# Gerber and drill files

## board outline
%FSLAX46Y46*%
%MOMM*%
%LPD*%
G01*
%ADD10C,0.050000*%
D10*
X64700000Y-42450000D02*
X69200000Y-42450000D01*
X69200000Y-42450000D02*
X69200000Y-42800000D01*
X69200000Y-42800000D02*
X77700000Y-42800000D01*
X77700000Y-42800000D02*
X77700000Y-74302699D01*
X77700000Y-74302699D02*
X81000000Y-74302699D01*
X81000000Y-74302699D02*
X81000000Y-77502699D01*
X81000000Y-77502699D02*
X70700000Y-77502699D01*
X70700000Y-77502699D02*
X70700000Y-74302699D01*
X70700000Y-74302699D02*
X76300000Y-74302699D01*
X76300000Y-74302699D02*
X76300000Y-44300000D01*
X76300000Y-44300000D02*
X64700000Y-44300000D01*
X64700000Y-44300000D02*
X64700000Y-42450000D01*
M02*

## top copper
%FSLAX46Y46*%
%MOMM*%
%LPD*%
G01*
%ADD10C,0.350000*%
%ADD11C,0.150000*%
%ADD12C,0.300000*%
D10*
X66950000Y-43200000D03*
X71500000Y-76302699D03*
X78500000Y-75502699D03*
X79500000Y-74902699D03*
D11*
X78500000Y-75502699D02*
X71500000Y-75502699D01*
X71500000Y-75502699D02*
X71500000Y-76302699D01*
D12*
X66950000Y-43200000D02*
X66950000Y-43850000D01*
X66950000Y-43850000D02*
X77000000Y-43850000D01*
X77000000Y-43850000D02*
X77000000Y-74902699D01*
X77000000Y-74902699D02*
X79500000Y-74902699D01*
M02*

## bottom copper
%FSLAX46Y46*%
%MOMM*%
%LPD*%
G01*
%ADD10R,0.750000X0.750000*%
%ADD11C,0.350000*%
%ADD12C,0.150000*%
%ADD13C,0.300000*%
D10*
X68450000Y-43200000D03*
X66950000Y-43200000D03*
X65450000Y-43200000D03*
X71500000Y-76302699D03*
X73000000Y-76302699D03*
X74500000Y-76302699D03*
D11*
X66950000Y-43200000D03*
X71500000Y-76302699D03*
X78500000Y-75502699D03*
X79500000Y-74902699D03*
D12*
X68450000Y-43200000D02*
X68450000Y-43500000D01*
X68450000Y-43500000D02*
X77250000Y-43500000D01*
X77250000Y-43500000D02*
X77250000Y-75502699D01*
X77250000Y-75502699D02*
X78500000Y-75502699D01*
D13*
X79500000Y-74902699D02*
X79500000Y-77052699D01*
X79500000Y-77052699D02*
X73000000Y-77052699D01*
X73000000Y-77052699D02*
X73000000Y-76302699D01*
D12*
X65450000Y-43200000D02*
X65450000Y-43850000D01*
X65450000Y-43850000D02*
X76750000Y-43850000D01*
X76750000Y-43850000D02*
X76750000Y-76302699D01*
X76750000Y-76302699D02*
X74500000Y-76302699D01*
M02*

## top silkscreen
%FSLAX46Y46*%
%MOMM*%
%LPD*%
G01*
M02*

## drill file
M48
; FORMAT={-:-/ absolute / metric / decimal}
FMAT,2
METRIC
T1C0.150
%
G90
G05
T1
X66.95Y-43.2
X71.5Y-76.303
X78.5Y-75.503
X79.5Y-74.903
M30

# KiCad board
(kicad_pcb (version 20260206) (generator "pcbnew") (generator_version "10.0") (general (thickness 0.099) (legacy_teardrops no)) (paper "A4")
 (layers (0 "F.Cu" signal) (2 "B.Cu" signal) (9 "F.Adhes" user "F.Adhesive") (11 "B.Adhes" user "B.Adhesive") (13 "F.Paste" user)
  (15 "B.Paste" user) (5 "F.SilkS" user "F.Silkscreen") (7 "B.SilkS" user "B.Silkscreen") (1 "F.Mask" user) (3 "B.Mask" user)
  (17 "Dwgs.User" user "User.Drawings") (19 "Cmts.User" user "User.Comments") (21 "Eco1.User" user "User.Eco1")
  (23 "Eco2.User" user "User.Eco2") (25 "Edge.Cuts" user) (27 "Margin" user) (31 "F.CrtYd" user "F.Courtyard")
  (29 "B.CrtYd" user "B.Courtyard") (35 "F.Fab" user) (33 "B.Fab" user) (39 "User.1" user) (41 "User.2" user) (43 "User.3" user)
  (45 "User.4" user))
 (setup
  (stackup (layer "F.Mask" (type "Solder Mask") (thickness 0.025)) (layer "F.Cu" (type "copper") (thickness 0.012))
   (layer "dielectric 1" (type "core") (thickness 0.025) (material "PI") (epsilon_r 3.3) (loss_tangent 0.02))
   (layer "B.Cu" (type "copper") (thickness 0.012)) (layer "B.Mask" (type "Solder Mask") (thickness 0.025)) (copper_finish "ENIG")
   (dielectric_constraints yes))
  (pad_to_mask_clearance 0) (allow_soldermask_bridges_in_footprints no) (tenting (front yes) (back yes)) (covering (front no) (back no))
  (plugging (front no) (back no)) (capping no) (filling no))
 (gr_line (start 64.7 42.45000000000001) (end 69.2 42.45000000000001) (stroke (width 0.05) (type default)) (layer "Edge.Cuts"))
 (gr_line (start 69.2 42.45000000000001) (end 69.2 42.80000000000001) (stroke (width 0.05) (type default)) (layer "Edge.Cuts"))
 (gr_line (start 69.2 42.80000000000001) (end 77.7 42.80000000000001) (stroke (width 0.05) (type default)) (layer "Edge.Cuts"))
 (gr_line (start 77.7 42.80000000000001) (end 77.7 74.30269878025518) (stroke (width 0.05) (type default)) (layer "Edge.Cuts"))
 (gr_line (start 77.7 74.30269878025518) (end 81.0 74.30269878025518) (stroke (width 0.05) (type default)) (layer "Edge.Cuts"))
 (gr_line (start 81.0 74.30269878025518) (end 81.0 77.50269878025519) (stroke (width 0.05) (type default)) (layer "Edge.Cuts"))
 (gr_line (start 81.0 77.50269878025519) (end 70.7 77.50269878025519) (stroke (width 0.05) (type default)) (layer "Edge.Cuts"))
 (gr_line (start 70.7 77.50269878025519) (end 70.7 74.30269878025518) (stroke (width 0.05) (type default)) (layer "Edge.Cuts"))
 (gr_line (start 70.7 74.30269878025518) (end 76.3 74.30269878025518) (stroke (width 0.05) (type default)) (layer "Edge.Cuts"))
 (gr_line (start 76.3 74.30269878025518) (end 76.3 44.3) (stroke (width 0.05) (type default)) (layer "Edge.Cuts"))
 (gr_line (start 76.3 44.3) (end 64.7 44.3) (stroke (width 0.05) (type default)) (layer "Edge.Cuts"))
 (gr_line (start 64.7 44.3) (end 64.7 42.45000000000001) (stroke (width 0.05) (type default)) (layer "Edge.Cuts"))
 (via (at 66.95 43.2) (size 0.35) (drill 0.15) (layers "F.Cu" "B.Cu") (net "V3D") (locked yes))
 (via (at 71.5 76.30269878025518) (size 0.35) (drill 0.15) (layers "F.Cu" "B.Cu") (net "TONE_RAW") (locked yes))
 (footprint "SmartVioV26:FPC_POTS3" (layer "F.Cu") (at 0 0)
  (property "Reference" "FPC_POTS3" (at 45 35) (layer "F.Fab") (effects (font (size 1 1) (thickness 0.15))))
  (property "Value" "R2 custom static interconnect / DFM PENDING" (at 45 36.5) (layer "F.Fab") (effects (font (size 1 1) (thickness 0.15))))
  (pad "S1" smd rect (at 68.45 43.2) (size 0.75 0.75) (layers "B.Cu" "B.Mask") (solder_mask_margin 0.1) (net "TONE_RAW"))
  (pad "S2" smd rect (at 66.95 43.2) (size 0.75 0.75) (layers "B.Cu" "B.Mask") (solder_mask_margin 0.1) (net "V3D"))
  (pad "S3" smd rect (at 65.45 43.2) (size 0.75 0.75) (layers "B.Cu" "B.Mask") (solder_mask_margin 0.1) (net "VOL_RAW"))
  (pad "T1" smd rect (at 71.5 76.30269878025518) (size 0.75 0.75) (layers "B.Cu" "B.Mask") (solder_mask_margin 0.1) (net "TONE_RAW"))
  (pad "T2" smd rect (at 73.0 76.30269878025518) (size 0.75 0.75) (layers "B.Cu" "B.Mask") (solder_mask_margin 0.1) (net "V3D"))
  (pad "T3" smd rect (at 74.5 76.30269878025518) (size 0.75 0.75) (layers "B.Cu" "B.Mask") (solder_mask_margin 0.1) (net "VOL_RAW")))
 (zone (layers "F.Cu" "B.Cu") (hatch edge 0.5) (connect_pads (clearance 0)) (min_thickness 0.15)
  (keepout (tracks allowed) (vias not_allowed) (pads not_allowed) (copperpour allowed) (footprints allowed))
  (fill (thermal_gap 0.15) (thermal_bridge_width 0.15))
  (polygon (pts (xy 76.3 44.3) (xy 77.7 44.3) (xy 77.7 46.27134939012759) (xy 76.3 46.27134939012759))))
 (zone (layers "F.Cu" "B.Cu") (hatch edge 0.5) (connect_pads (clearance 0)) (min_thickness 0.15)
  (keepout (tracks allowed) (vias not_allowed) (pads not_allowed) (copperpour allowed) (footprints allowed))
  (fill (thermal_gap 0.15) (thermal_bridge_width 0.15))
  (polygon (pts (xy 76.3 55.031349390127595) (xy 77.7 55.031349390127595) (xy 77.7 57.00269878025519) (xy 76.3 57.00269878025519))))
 (segment (start 68.45 43.2) (end 68.45 43.5) (width 0.15) (layer "B.Cu") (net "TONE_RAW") (locked yes))
 (segment (start 68.45 43.5) (end 77.25 43.5) (width 0.15) (layer "B.Cu") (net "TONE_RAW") (locked yes))
 (segment (start 77.25 43.5) (end 77.25 75.50269878025519) (width 0.15) (layer "B.Cu") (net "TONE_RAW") (locked yes))
 (segment (start 77.25 75.50269878025519) (end 78.5 75.50269878025519) (width 0.15) (layer "B.Cu") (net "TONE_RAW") (locked yes))
 (segment (start 78.5 75.50269878025519) (end 71.5 75.50269878025519) (width 0.15) (layer "F.Cu") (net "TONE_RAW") (locked yes))
 (segment (start 71.5 75.50269878025519) (end 71.5 76.30269878025518) (width 0.15) (layer "F.Cu") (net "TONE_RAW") (locked yes))
 (via (at 78.5 75.50269878025519) (size 0.35) (drill 0.15) (layers "F.Cu" "B.Cu") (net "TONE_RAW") (locked yes))
 (segment (start 66.95 43.2) (end 66.95 43.85) (width 0.3) (layer "F.Cu") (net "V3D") (locked yes))
 (segment (start 66.95 43.85) (end 77.0 43.85) (width 0.3) (layer "F.Cu") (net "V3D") (locked yes))
 (segment (start 77.0 43.85) (end 77.0 74.90269878025518) (width 0.3) (layer "F.Cu") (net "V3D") (locked yes))
 (segment (start 77.0 74.90269878025518) (end 79.5 74.90269878025518) (width 0.3) (layer "F.Cu") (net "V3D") (locked yes))
 (segment (start 79.5 74.90269878025518) (end 79.5 77.05269878025518) (width 0.3) (layer "B.Cu") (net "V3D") (locked yes))
 (segment (start 79.5 77.05269878025518) (end 73.0 77.05269878025518) (width 0.3) (layer "B.Cu") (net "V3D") (locked yes))
 (segment (start 73.0 77.05269878025518) (end 73.0 76.30269878025518) (width 0.3) (layer "B.Cu") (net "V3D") (locked yes))
 (via (at 79.5 74.90269878025518) (size 0.35) (drill 0.15) (layers "F.Cu" "B.Cu") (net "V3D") (locked yes))
 (segment (start 65.45 43.2) (end 65.45 43.85) (width 0.15) (layer "B.Cu") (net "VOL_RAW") (locked yes))
 (segment (start 65.45 43.85) (end 76.75 43.85) (width 0.15) (layer "B.Cu") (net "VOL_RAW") (locked yes))
 (segment (start 76.75 43.85) (end 76.75 76.30269878025518) (width 0.15) (layer "B.Cu") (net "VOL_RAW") (locked yes))
 (segment (start 76.75 76.30269878025518) (end 74.5 76.30269878025518) (width 0.15) (layer "B.Cu") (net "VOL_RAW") (locked yes)))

